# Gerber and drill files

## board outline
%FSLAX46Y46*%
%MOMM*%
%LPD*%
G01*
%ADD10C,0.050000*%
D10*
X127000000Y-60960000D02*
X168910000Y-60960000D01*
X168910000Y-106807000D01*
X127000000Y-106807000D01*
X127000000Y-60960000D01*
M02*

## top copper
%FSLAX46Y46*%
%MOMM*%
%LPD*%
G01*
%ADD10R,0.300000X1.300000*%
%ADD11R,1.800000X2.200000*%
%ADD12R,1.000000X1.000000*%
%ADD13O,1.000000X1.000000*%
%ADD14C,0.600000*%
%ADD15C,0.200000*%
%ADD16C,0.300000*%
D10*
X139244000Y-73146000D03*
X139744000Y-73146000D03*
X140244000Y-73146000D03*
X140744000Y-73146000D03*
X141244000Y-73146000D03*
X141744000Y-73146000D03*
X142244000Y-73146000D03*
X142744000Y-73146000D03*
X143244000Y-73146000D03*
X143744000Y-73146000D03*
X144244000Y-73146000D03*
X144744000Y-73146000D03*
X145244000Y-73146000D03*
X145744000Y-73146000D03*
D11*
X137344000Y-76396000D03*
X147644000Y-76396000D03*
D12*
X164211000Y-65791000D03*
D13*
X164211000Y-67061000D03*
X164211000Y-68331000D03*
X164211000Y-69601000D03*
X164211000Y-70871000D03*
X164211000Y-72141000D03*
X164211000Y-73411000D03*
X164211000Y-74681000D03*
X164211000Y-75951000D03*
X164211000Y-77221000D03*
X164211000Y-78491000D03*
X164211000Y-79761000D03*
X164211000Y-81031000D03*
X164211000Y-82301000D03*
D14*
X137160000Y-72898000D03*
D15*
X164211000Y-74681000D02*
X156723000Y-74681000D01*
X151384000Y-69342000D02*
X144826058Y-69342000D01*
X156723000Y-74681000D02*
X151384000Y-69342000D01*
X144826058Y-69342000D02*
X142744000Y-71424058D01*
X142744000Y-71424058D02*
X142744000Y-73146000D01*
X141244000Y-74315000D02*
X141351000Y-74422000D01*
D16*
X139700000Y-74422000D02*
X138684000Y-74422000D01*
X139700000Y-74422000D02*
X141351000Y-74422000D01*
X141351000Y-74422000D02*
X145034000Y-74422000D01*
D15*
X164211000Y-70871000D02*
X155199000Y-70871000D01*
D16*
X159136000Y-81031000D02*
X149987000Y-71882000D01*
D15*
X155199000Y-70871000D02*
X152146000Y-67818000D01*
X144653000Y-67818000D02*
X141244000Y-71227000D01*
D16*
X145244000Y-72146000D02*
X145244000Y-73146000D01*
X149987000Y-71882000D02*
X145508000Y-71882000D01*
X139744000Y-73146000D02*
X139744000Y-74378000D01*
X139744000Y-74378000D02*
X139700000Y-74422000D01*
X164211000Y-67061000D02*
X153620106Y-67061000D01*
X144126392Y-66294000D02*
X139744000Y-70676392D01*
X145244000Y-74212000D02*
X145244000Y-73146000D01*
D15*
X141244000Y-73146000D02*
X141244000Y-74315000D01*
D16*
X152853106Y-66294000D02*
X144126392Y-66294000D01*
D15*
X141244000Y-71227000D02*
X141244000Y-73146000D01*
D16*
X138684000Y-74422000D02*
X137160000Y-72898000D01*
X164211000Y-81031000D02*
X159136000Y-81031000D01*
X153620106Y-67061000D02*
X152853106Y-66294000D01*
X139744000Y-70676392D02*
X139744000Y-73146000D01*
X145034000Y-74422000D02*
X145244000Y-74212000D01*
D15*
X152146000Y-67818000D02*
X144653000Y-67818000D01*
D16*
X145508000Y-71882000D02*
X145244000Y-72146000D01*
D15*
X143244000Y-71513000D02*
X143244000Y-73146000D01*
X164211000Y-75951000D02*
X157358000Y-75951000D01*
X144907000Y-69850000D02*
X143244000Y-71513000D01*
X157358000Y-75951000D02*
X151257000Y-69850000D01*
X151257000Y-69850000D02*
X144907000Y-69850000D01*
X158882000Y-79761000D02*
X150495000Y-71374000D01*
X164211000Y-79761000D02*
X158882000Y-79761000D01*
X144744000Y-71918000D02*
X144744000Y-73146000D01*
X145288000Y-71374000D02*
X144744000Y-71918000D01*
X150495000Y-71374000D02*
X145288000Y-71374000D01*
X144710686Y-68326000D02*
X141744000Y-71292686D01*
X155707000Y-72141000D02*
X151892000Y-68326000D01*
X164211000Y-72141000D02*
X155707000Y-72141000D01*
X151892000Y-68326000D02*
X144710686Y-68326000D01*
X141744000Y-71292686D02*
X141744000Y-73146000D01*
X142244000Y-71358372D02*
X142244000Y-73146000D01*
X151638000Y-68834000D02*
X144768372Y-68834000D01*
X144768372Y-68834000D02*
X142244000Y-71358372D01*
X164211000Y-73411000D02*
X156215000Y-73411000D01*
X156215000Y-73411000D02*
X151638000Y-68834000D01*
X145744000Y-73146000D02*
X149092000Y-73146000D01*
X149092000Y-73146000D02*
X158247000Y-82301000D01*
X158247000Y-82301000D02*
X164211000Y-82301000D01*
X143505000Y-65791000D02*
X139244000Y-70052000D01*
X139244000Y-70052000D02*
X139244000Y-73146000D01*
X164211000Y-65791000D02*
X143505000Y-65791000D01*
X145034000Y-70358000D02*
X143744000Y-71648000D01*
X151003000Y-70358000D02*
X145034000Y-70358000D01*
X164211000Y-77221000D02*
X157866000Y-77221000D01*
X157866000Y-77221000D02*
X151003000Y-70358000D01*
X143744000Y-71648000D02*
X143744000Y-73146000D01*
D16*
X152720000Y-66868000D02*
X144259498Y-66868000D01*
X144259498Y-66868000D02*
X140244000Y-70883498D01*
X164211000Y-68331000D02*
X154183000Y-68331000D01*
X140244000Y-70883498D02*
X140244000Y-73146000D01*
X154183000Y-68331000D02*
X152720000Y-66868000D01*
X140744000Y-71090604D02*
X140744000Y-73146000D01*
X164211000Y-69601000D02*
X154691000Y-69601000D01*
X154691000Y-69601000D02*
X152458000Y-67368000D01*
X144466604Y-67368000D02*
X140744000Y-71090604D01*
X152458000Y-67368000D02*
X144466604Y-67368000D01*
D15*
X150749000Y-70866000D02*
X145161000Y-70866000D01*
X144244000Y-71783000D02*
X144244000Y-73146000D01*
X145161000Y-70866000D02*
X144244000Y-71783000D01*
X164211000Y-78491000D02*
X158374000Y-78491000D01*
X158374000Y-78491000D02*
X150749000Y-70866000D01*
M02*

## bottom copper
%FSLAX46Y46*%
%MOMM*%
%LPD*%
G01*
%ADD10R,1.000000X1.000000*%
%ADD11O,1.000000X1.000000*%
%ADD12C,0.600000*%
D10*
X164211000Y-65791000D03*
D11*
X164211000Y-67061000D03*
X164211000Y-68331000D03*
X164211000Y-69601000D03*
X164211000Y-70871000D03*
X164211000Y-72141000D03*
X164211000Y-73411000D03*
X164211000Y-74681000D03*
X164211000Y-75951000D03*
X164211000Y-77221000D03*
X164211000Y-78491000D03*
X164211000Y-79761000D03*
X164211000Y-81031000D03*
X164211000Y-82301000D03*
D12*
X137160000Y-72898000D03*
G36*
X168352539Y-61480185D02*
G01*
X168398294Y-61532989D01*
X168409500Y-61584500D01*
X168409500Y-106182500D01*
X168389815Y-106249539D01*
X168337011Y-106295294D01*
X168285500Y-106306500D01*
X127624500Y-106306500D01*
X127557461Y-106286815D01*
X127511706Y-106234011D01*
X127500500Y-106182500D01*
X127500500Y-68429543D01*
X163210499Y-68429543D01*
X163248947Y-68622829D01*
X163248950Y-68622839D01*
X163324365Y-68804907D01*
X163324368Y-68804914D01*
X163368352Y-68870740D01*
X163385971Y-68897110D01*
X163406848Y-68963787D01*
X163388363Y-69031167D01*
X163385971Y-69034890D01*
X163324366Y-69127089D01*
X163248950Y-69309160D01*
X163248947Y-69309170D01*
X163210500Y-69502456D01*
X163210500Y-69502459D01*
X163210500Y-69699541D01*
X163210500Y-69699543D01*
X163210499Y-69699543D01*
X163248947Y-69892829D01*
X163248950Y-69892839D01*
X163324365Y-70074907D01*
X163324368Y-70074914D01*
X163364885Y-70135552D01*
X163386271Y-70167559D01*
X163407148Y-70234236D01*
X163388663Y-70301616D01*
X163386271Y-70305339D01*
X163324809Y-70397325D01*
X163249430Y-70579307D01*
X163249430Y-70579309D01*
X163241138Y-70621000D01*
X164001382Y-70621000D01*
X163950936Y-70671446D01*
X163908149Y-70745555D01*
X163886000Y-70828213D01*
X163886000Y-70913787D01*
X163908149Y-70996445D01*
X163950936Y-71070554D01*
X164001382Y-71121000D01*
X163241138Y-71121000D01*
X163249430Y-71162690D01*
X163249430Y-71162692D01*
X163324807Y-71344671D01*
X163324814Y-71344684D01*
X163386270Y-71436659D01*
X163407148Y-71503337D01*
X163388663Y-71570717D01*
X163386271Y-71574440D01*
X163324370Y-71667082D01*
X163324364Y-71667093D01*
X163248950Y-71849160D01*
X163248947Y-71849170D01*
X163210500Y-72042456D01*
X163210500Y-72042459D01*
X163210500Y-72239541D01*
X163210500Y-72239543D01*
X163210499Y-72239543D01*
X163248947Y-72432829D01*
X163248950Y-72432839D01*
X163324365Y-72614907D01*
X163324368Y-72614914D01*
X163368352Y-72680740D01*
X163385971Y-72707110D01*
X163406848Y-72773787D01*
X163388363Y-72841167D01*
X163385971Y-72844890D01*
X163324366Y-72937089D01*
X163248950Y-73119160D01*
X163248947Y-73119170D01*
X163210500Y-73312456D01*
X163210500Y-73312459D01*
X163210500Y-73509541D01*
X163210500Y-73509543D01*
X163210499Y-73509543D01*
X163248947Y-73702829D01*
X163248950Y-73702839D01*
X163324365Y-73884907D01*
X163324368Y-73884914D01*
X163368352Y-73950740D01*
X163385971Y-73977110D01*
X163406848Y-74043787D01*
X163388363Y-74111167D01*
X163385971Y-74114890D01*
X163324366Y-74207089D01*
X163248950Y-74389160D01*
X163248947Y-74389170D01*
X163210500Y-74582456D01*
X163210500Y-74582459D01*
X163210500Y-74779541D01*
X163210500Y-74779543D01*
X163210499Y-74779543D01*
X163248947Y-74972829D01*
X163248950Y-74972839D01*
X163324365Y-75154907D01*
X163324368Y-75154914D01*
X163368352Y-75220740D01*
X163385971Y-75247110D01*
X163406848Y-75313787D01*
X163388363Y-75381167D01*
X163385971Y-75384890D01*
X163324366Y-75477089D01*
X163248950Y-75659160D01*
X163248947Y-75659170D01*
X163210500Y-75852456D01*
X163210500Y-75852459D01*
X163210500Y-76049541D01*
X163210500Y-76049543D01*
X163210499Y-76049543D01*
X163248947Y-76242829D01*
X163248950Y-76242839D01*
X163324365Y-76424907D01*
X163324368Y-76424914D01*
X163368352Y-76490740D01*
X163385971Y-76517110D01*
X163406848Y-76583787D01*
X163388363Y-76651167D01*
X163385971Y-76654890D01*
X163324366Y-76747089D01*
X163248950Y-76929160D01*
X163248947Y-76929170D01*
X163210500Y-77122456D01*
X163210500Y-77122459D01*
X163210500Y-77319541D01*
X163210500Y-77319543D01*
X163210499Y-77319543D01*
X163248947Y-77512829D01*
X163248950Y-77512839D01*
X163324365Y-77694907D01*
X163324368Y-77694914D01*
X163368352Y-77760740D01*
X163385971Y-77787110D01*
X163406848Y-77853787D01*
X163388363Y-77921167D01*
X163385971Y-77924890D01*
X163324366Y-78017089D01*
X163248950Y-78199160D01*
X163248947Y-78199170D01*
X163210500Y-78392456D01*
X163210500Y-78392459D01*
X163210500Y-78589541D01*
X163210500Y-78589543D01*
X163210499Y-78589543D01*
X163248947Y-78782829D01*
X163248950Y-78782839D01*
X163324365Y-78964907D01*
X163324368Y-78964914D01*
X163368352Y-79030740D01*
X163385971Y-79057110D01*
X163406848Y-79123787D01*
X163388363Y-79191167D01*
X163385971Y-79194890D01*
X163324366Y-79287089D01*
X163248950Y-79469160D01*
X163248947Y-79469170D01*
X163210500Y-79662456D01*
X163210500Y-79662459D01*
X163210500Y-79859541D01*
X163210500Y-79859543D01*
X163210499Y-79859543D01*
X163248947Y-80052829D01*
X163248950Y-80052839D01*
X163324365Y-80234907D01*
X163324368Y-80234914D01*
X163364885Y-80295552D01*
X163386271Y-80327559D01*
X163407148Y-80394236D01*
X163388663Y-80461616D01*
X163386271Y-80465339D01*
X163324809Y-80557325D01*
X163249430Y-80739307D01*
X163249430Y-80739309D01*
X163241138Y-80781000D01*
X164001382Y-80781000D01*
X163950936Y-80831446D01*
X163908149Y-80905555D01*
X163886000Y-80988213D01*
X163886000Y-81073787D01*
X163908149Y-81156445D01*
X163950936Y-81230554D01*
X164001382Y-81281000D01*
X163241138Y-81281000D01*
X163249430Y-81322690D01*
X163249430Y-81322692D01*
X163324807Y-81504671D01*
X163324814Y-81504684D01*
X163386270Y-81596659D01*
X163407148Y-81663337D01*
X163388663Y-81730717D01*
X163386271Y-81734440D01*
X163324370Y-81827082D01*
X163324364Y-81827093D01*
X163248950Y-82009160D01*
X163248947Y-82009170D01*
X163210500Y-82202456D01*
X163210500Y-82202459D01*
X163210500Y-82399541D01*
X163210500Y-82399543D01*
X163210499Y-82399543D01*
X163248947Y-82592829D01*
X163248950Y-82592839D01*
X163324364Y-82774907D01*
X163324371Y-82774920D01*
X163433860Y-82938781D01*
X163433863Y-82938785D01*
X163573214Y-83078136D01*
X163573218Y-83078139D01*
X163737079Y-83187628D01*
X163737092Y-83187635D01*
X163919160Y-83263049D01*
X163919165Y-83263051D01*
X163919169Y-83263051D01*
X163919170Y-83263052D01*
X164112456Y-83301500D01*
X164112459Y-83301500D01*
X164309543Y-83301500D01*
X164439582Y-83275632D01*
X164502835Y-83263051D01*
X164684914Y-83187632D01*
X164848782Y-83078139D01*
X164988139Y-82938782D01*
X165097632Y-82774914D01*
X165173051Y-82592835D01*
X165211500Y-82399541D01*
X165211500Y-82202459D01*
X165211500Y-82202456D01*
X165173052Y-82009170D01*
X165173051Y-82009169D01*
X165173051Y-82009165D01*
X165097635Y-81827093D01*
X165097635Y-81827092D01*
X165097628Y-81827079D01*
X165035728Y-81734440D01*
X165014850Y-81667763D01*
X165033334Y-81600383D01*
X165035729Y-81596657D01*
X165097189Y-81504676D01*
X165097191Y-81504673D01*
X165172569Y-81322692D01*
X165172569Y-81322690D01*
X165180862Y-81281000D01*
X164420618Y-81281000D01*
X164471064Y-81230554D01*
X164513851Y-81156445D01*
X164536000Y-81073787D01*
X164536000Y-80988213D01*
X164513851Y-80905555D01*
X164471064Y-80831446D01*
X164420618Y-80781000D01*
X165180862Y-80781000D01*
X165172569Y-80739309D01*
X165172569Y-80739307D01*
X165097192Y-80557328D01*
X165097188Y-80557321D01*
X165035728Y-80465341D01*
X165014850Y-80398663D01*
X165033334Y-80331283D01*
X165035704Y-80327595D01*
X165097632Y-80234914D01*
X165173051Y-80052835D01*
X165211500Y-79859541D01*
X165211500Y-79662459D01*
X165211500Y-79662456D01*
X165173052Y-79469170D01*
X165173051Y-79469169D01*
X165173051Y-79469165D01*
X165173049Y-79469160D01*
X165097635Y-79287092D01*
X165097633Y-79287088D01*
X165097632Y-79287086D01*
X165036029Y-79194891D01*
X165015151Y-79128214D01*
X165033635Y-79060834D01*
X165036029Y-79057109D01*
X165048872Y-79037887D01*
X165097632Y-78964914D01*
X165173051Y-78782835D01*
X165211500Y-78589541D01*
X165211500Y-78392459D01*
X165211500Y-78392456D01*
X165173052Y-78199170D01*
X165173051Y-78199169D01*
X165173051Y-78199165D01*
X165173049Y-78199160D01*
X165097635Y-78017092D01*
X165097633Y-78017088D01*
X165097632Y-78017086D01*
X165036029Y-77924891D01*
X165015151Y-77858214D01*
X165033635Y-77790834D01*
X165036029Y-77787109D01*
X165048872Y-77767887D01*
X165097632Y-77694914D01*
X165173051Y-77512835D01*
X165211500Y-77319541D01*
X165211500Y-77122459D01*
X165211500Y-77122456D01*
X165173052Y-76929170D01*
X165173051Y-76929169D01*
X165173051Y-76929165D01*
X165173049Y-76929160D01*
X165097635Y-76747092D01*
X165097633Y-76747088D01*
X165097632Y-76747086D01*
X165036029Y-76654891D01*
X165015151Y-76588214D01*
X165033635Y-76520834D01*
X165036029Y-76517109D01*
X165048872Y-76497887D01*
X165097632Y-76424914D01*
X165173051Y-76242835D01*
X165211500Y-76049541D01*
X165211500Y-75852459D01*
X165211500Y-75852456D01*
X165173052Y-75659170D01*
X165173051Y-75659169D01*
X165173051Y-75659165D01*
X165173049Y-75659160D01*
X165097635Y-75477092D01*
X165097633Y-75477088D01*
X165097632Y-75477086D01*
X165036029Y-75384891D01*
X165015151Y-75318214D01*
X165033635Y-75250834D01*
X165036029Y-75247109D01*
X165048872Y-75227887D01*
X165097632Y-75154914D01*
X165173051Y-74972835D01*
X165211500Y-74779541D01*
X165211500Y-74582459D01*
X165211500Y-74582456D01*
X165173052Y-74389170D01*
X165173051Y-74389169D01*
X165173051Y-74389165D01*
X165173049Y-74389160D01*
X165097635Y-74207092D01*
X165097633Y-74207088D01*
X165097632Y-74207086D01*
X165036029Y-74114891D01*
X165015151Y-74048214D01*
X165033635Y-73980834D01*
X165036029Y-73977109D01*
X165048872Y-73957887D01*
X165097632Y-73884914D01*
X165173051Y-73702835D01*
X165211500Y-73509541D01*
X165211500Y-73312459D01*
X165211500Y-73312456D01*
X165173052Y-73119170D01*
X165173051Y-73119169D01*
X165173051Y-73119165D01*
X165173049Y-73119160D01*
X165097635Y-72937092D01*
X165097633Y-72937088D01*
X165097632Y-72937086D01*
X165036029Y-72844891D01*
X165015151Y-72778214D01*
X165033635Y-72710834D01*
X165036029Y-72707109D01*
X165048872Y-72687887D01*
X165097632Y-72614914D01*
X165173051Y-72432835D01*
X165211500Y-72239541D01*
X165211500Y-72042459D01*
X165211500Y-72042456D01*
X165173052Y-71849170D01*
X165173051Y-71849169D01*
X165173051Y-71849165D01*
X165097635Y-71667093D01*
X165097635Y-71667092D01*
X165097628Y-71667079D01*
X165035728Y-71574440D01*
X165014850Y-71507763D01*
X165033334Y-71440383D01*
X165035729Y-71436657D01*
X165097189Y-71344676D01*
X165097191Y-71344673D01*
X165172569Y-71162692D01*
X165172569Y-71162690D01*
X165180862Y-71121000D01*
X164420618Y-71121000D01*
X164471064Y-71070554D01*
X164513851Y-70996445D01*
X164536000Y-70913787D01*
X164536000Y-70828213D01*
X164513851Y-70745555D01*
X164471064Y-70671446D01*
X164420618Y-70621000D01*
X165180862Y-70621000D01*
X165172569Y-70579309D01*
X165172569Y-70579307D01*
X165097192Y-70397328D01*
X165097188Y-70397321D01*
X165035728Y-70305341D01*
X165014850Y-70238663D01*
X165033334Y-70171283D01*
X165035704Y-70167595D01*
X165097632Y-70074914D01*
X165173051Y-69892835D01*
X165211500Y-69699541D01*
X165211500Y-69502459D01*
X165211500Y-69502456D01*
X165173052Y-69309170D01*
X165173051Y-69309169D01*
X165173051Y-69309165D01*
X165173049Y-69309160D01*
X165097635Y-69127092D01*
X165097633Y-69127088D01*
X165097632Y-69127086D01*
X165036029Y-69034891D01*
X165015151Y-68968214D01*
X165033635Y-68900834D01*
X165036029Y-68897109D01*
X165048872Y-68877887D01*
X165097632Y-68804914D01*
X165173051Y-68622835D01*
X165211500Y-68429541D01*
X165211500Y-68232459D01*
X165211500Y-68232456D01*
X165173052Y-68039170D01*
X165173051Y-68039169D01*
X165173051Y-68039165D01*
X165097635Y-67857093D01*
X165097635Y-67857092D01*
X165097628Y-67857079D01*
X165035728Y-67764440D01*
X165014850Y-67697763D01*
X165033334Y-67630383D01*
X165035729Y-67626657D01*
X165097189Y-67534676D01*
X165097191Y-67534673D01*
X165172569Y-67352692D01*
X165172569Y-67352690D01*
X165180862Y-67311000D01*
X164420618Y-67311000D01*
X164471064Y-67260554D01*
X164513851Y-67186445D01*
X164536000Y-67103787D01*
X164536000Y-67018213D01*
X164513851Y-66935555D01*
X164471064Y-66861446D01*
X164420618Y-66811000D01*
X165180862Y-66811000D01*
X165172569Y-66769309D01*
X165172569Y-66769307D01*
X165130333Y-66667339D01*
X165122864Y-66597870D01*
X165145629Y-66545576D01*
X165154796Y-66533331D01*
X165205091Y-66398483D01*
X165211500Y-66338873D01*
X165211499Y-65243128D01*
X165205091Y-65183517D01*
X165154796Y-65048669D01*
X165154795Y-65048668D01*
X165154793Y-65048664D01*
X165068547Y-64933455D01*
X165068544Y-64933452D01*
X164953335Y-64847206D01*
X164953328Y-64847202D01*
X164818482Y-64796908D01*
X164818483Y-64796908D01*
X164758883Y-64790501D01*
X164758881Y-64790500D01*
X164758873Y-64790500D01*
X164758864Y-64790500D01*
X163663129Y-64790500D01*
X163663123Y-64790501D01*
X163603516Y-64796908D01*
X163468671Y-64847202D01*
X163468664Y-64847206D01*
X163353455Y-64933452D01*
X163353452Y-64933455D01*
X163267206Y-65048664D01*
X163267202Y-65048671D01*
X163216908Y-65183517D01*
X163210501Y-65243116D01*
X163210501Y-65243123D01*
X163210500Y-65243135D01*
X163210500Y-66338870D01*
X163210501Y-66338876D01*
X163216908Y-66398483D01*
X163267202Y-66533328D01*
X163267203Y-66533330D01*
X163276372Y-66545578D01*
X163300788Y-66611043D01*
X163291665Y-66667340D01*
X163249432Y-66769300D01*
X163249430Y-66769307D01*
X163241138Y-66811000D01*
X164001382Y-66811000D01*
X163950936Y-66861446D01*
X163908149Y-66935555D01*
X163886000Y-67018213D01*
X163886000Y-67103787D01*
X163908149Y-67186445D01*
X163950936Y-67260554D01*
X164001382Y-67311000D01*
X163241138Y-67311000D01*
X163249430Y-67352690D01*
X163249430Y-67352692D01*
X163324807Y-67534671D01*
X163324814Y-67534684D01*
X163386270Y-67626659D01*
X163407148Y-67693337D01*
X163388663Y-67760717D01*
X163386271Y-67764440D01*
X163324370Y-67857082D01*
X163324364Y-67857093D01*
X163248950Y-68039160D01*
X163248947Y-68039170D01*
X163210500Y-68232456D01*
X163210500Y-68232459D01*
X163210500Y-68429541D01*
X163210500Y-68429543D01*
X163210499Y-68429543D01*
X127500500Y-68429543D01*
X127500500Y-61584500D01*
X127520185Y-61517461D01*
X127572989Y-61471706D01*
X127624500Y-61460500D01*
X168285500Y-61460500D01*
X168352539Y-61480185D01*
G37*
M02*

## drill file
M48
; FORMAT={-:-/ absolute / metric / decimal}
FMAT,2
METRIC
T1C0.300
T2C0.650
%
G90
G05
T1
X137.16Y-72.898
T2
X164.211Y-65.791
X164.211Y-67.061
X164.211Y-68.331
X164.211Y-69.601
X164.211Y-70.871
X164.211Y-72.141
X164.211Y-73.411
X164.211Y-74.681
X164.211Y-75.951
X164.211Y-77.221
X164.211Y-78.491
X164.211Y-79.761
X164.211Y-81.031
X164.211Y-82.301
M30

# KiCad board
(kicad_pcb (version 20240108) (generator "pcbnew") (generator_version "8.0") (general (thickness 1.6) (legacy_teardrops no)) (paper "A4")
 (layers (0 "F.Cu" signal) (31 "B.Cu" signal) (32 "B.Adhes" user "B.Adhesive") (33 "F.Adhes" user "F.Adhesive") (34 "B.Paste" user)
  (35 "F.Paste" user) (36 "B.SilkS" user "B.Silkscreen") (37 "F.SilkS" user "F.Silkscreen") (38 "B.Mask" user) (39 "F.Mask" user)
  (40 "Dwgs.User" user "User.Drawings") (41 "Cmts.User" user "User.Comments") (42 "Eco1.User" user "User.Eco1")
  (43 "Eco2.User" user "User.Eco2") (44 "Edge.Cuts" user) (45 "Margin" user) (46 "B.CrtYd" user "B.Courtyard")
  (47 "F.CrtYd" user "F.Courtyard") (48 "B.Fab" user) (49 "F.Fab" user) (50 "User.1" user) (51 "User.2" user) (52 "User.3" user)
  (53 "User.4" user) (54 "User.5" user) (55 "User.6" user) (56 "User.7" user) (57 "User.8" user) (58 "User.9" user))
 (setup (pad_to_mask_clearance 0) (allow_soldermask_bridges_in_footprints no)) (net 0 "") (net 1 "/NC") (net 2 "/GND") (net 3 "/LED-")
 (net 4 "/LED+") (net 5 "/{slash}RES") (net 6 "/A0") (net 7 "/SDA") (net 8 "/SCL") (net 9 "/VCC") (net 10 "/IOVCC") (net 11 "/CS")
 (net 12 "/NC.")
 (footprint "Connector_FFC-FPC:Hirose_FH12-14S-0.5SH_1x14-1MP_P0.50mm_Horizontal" (layer "F.Cu") (at 142.494 74.996)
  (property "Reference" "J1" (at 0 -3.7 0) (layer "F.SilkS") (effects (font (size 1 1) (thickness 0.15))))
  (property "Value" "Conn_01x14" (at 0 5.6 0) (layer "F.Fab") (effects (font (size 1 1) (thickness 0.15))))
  (pad "1" smd rect (at -3.25 -1.85) (size 0.3 1.3) (layers "F.Cu" "F.Paste" "F.Mask") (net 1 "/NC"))
  (pad "2" smd rect (at -2.75 -1.85) (size 0.3 1.3) (layers "F.Cu" "F.Paste" "F.Mask") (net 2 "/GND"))
  (pad "3" smd rect (at -2.25 -1.85) (size 0.3 1.3) (layers "F.Cu" "F.Paste" "F.Mask") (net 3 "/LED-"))
  (pad "4" smd rect (at -1.75 -1.85) (size 0.3 1.3) (layers "F.Cu" "F.Paste" "F.Mask") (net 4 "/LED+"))
  (pad "5" smd rect (at -1.25 -1.85) (size 0.3 1.3) (layers "F.Cu" "F.Paste" "F.Mask") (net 2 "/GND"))
  (pad "6" smd rect (at -0.75 -1.85) (size 0.3 1.3) (layers "F.Cu" "F.Paste" "F.Mask") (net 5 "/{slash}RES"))
  (pad "7" smd rect (at -0.25 -1.85) (size 0.3 1.3) (layers "F.Cu" "F.Paste" "F.Mask") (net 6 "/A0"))
  (pad "8" smd rect (at 0.25 -1.85) (size 0.3 1.3) (layers "F.Cu" "F.Paste" "F.Mask") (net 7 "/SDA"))
  (pad "9" smd rect (at 0.75 -1.85) (size 0.3 1.3) (layers "F.Cu" "F.Paste" "F.Mask") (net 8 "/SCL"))
  (pad "10" smd rect (at 1.25 -1.85) (size 0.3 1.3) (layers "F.Cu" "F.Paste" "F.Mask") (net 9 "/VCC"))
  (pad "11" smd rect (at 1.75 -1.85) (size 0.3 1.3) (layers "F.Cu" "F.Paste" "F.Mask") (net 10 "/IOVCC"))
  (pad "12" smd rect (at 2.25 -1.85) (size 0.3 1.3) (layers "F.Cu" "F.Paste" "F.Mask") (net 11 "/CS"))
  (pad "13" smd rect (at 2.75 -1.85) (size 0.3 1.3) (layers "F.Cu" "F.Paste" "F.Mask") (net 2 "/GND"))
  (pad "14" smd rect (at 3.25 -1.85) (size 0.3 1.3) (layers "F.Cu" "F.Paste" "F.Mask") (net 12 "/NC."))
  (pad "MP" smd rect (at -5.15 1.4) (size 1.8 2.2) (layers "F.Cu" "F.Paste" "F.Mask"))
  (pad "MP" smd rect (at 5.15 1.4) (size 1.8 2.2) (layers "F.Cu" "F.Paste" "F.Mask")))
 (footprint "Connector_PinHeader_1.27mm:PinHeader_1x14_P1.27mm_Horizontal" (layer "F.Cu") (at 164.211 65.791)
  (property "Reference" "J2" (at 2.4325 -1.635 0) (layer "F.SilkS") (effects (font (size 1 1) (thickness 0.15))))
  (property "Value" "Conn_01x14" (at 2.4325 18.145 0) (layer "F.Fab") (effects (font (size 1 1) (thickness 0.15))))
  (pad "1" thru_hole rect (at 0 0) (size 1 1) (drill 0.65) (layers "*.Cu" "*.Mask") (remove_unused_layers no) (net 1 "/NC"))
  (pad "2" thru_hole oval (at 0 1.27) (size 1 1) (drill 0.65) (layers "*.Cu" "*.Mask") (remove_unused_layers no) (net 2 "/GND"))
  (pad "3" thru_hole oval (at 0 2.54) (size 1 1) (drill 0.65) (layers "*.Cu" "*.Mask") (remove_unused_layers no) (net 3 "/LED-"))
  (pad "4" thru_hole oval (at 0 3.81) (size 1 1) (drill 0.65) (layers "*.Cu" "*.Mask") (remove_unused_layers no) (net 4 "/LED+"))
  (pad "5" thru_hole oval (at 0 5.08) (size 1 1) (drill 0.65) (layers "*.Cu" "*.Mask") (remove_unused_layers no) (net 2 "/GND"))
  (pad "6" thru_hole oval (at 0 6.35) (size 1 1) (drill 0.65) (layers "*.Cu" "*.Mask") (remove_unused_layers no) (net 5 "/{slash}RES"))
  (pad "7" thru_hole oval (at 0 7.62) (size 1 1) (drill 0.65) (layers "*.Cu" "*.Mask") (remove_unused_layers no) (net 6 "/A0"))
  (pad "8" thru_hole oval (at 0 8.89) (size 1 1) (drill 0.65) (layers "*.Cu" "*.Mask") (remove_unused_layers no) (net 7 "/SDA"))
  (pad "9" thru_hole oval (at 0 10.16) (size 1 1) (drill 0.65) (layers "*.Cu" "*.Mask") (remove_unused_layers no) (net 8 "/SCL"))
  (pad "10" thru_hole oval (at 0 11.43) (size 1 1) (drill 0.65) (layers "*.Cu" "*.Mask") (remove_unused_layers no) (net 9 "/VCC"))
  (pad "11" thru_hole oval (at 0 12.7) (size 1 1) (drill 0.65) (layers "*.Cu" "*.Mask") (remove_unused_layers no) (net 10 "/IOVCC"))
  (pad "12" thru_hole oval (at 0 13.97) (size 1 1) (drill 0.65) (layers "*.Cu" "*.Mask") (remove_unused_layers no) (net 11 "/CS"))
  (pad "13" thru_hole oval (at 0 15.24) (size 1 1) (drill 0.65) (layers "*.Cu" "*.Mask") (remove_unused_layers no) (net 2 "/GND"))
  (pad "14" thru_hole oval (at 0 16.51) (size 1 1) (drill 0.65) (layers "*.Cu" "*.Mask") (remove_unused_layers no) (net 12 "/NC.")))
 (gr_rect (start 127 60.96) (end 168.91 106.807) (stroke (width 0.05) (type default)) (fill none) (layer "Edge.Cuts"))
 (segment (start 164.211 74.681) (end 156.723 74.681) (width 0.2) (layer "F.Cu") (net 7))
 (segment (start 151.384 69.342) (end 144.826058 69.342) (width 0.2) (layer "F.Cu") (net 7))
 (segment (start 156.723 74.681) (end 151.384 69.342) (width 0.2) (layer "F.Cu") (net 7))
 (segment (start 144.826058 69.342) (end 142.744 71.424058) (width 0.2) (layer "F.Cu") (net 7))
 (segment (start 142.744 71.424058) (end 142.744 73.146) (width 0.2) (layer "F.Cu") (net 7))
 (segment (start 141.244 74.315) (end 141.351 74.422) (width 0.2) (layer "F.Cu") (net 2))
 (segment (start 139.7 74.422) (end 138.684 74.422) (width 0.3) (layer "F.Cu") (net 2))
 (segment (start 139.7 74.422) (end 141.351 74.422) (width 0.3) (layer "F.Cu") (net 2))
 (segment (start 141.351 74.422) (end 145.034 74.422) (width 0.3) (layer "F.Cu") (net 2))
 (segment (start 164.211 70.871) (end 155.199 70.871) (width 0.2) (layer "F.Cu") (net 2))
 (segment (start 159.136 81.031) (end 149.987 71.882) (width 0.3) (layer "F.Cu") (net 2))
 (segment (start 155.199 70.871) (end 152.146 67.818) (width 0.2) (layer "F.Cu") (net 2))
 (segment (start 144.653 67.818) (end 141.244 71.227) (width 0.2) (layer "F.Cu") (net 2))
 (segment (start 145.244 72.146) (end 145.244 73.146) (width 0.3) (layer "F.Cu") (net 2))
 (segment (start 149.987 71.882) (end 145.508 71.882) (width 0.3) (layer "F.Cu") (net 2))
 (segment (start 139.744 73.146) (end 139.744 74.378) (width 0.3) (layer "F.Cu") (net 2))
 (segment (start 139.744 74.378) (end 139.7 74.422) (width 0.3) (layer "F.Cu") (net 2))
 (segment (start 164.211 67.061) (end 153.620106 67.061) (width 0.3) (layer "F.Cu") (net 2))
 (segment (start 144.126392 66.294) (end 139.744 70.676392) (width 0.3) (layer "F.Cu") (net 2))
 (segment (start 145.244 74.212) (end 145.244 73.146) (width 0.3) (layer "F.Cu") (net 2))
 (segment (start 141.244 73.146) (end 141.244 74.315) (width 0.2) (layer "F.Cu") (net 2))
 (segment (start 152.853106 66.294) (end 144.126392 66.294) (width 0.3) (layer "F.Cu") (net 2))
 (segment (start 141.244 71.227) (end 141.244 73.146) (width 0.2) (layer "F.Cu") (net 2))
 (segment (start 138.684 74.422) (end 137.16 72.898) (width 0.3) (layer "F.Cu") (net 2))
 (segment (start 164.211 81.031) (end 159.136 81.031) (width 0.3) (layer "F.Cu") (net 2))
 (segment (start 153.620106 67.061) (end 152.853106 66.294) (width 0.3) (layer "F.Cu") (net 2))
 (segment (start 139.744 70.676392) (end 139.744 73.146) (width 0.3) (layer "F.Cu") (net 2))
 (segment (start 145.034 74.422) (end 145.244 74.212) (width 0.3) (layer "F.Cu") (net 2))
 (segment (start 152.146 67.818) (end 144.653 67.818) (width 0.2) (layer "F.Cu") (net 2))
 (segment (start 145.508 71.882) (end 145.244 72.146) (width 0.3) (layer "F.Cu") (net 2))
 (via (at 137.16 72.898) (size 0.6) (drill 0.3) (layers "F.Cu" "B.Cu") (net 2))
 (segment (start 143.244 71.513) (end 143.244 73.146) (width 0.2) (layer "F.Cu") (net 8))
 (segment (start 164.211 75.951) (end 157.358 75.951) (width 0.2) (layer "F.Cu") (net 8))
 (segment (start 144.907 69.85) (end 143.244 71.513) (width 0.2) (layer "F.Cu") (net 8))
 (segment (start 157.358 75.951) (end 151.257 69.85) (width 0.2) (layer "F.Cu") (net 8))
 (segment (start 151.257 69.85) (end 144.907 69.85) (width 0.2) (layer "F.Cu") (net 8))
 (segment (start 158.882 79.761) (end 150.495 71.374) (width 0.2) (layer "F.Cu") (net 11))
 (segment (start 164.211 79.761) (end 158.882 79.761) (width 0.2) (layer "F.Cu") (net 11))
 (segment (start 144.744 71.918) (end 144.744 73.146) (width 0.2) (layer "F.Cu") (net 11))
 (segment (start 145.288 71.374) (end 144.744 71.918) (width 0.2) (layer "F.Cu") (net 11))
 (segment (start 150.495 71.374) (end 145.288 71.374) (width 0.2) (layer "F.Cu") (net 11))
 (segment (start 144.710686 68.326) (end 141.744 71.292686) (width 0.2) (layer "F.Cu") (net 5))
 (segment (start 155.707 72.141) (end 151.892 68.326) (width 0.2) (layer "F.Cu") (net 5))
 (segment (start 164.211 72.141) (end 155.707 72.141) (width 0.2) (layer "F.Cu") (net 5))
 (segment (start 151.892 68.326) (end 144.710686 68.326) (width 0.2) (layer "F.Cu") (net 5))
 (segment (start 141.744 71.292686) (end 141.744 73.146) (width 0.2) (layer "F.Cu") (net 5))
 (segment (start 142.244 71.358372) (end 142.244 73.146) (width 0.2) (layer "F.Cu") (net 6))
 (segment (start 151.638 68.834) (end 144.768372 68.834) (width 0.2) (layer "F.Cu") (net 6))
 (segment (start 144.768372 68.834) (end 142.244 71.358372) (width 0.2) (layer "F.Cu") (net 6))
 (segment (start 164.211 73.411) (end 156.215 73.411) (width 0.2) (layer "F.Cu") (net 6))
 (segment (start 156.215 73.411) (end 151.638 68.834) (width 0.2) (layer "F.Cu") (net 6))
 (segment (start 145.744 73.146) (end 149.092 73.146) (width 0.2) (layer "F.Cu") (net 12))
 (segment (start 149.092 73.146) (end 158.247 82.301) (width 0.2) (layer "F.Cu") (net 12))
 (segment (start 158.247 82.301) (end 164.211 82.301) (width 0.2) (layer "F.Cu") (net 12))
 (segment (start 143.505 65.791) (end 139.244 70.052) (width 0.2) (layer "F.Cu") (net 1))
 (segment (start 139.244 70.052) (end 139.244 73.146) (width 0.2) (layer "F.Cu") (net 1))
 (segment (start 164.211 65.791) (end 143.505 65.791) (width 0.2) (layer "F.Cu") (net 1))
 (segment (start 145.034 70.358) (end 143.744 71.648) (width 0.2) (layer "F.Cu") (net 9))
 (segment (start 151.003 70.358) (end 145.034 70.358) (width 0.2) (layer "F.Cu") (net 9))
 (segment (start 164.211 77.221) (end 157.866 77.221) (width 0.2) (layer "F.Cu") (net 9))
 (segment (start 157.866 77.221) (end 151.003 70.358) (width 0.2) (layer "F.Cu") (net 9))
 (segment (start 143.744 71.648) (end 143.744 73.146) (width 0.2) (layer "F.Cu") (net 9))
 (segment (start 152.72 66.868) (end 144.259498 66.868) (width 0.3) (layer "F.Cu") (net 3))
 (segment (start 144.259498 66.868) (end 140.244 70.883498) (width 0.3) (layer "F.Cu") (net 3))
 (segment (start 164.211 68.331) (end 154.183 68.331) (width 0.3) (layer "F.Cu") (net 3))
 (segment (start 140.244 70.883498) (end 140.244 73.146) (width 0.3) (layer "F.Cu") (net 3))
 (segment (start 154.183 68.331) (end 152.72 66.868) (width 0.3) (layer "F.Cu") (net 3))
 (segment (start 140.744 71.090604) (end 140.744 73.146) (width 0.3) (layer "F.Cu") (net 4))
 (segment (start 164.211 69.601) (end 154.691 69.601) (width 0.3) (layer "F.Cu") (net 4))
 (segment (start 154.691 69.601) (end 152.458 67.368) (width 0.3) (layer "F.Cu") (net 4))
 (segment (start 144.466604 67.368) (end 140.744 71.090604) (width 0.3) (layer "F.Cu") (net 4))
 (segment (start 152.458 67.368) (end 144.466604 67.368) (width 0.3) (layer "F.Cu") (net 4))
 (segment (start 150.749 70.866) (end 145.161 70.866) (width 0.2) (layer "F.Cu") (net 10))
 (segment (start 144.244 71.783) (end 144.244 73.146) (width 0.2) (layer "F.Cu") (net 10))
 (segment (start 145.161 70.866) (end 144.244 71.783) (width 0.2) (layer "F.Cu") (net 10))
 (segment (start 164.211 78.491) (end 158.374 78.491) (width 0.2) (layer "F.Cu") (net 10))
 (segment (start 158.374 78.491) (end 150.749 70.866) (width 0.2) (layer "F.Cu") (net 10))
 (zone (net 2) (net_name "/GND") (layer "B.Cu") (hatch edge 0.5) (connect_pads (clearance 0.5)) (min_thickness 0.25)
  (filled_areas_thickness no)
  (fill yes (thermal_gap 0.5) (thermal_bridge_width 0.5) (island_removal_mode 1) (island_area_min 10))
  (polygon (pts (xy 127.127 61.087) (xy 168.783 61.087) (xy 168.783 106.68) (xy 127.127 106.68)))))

